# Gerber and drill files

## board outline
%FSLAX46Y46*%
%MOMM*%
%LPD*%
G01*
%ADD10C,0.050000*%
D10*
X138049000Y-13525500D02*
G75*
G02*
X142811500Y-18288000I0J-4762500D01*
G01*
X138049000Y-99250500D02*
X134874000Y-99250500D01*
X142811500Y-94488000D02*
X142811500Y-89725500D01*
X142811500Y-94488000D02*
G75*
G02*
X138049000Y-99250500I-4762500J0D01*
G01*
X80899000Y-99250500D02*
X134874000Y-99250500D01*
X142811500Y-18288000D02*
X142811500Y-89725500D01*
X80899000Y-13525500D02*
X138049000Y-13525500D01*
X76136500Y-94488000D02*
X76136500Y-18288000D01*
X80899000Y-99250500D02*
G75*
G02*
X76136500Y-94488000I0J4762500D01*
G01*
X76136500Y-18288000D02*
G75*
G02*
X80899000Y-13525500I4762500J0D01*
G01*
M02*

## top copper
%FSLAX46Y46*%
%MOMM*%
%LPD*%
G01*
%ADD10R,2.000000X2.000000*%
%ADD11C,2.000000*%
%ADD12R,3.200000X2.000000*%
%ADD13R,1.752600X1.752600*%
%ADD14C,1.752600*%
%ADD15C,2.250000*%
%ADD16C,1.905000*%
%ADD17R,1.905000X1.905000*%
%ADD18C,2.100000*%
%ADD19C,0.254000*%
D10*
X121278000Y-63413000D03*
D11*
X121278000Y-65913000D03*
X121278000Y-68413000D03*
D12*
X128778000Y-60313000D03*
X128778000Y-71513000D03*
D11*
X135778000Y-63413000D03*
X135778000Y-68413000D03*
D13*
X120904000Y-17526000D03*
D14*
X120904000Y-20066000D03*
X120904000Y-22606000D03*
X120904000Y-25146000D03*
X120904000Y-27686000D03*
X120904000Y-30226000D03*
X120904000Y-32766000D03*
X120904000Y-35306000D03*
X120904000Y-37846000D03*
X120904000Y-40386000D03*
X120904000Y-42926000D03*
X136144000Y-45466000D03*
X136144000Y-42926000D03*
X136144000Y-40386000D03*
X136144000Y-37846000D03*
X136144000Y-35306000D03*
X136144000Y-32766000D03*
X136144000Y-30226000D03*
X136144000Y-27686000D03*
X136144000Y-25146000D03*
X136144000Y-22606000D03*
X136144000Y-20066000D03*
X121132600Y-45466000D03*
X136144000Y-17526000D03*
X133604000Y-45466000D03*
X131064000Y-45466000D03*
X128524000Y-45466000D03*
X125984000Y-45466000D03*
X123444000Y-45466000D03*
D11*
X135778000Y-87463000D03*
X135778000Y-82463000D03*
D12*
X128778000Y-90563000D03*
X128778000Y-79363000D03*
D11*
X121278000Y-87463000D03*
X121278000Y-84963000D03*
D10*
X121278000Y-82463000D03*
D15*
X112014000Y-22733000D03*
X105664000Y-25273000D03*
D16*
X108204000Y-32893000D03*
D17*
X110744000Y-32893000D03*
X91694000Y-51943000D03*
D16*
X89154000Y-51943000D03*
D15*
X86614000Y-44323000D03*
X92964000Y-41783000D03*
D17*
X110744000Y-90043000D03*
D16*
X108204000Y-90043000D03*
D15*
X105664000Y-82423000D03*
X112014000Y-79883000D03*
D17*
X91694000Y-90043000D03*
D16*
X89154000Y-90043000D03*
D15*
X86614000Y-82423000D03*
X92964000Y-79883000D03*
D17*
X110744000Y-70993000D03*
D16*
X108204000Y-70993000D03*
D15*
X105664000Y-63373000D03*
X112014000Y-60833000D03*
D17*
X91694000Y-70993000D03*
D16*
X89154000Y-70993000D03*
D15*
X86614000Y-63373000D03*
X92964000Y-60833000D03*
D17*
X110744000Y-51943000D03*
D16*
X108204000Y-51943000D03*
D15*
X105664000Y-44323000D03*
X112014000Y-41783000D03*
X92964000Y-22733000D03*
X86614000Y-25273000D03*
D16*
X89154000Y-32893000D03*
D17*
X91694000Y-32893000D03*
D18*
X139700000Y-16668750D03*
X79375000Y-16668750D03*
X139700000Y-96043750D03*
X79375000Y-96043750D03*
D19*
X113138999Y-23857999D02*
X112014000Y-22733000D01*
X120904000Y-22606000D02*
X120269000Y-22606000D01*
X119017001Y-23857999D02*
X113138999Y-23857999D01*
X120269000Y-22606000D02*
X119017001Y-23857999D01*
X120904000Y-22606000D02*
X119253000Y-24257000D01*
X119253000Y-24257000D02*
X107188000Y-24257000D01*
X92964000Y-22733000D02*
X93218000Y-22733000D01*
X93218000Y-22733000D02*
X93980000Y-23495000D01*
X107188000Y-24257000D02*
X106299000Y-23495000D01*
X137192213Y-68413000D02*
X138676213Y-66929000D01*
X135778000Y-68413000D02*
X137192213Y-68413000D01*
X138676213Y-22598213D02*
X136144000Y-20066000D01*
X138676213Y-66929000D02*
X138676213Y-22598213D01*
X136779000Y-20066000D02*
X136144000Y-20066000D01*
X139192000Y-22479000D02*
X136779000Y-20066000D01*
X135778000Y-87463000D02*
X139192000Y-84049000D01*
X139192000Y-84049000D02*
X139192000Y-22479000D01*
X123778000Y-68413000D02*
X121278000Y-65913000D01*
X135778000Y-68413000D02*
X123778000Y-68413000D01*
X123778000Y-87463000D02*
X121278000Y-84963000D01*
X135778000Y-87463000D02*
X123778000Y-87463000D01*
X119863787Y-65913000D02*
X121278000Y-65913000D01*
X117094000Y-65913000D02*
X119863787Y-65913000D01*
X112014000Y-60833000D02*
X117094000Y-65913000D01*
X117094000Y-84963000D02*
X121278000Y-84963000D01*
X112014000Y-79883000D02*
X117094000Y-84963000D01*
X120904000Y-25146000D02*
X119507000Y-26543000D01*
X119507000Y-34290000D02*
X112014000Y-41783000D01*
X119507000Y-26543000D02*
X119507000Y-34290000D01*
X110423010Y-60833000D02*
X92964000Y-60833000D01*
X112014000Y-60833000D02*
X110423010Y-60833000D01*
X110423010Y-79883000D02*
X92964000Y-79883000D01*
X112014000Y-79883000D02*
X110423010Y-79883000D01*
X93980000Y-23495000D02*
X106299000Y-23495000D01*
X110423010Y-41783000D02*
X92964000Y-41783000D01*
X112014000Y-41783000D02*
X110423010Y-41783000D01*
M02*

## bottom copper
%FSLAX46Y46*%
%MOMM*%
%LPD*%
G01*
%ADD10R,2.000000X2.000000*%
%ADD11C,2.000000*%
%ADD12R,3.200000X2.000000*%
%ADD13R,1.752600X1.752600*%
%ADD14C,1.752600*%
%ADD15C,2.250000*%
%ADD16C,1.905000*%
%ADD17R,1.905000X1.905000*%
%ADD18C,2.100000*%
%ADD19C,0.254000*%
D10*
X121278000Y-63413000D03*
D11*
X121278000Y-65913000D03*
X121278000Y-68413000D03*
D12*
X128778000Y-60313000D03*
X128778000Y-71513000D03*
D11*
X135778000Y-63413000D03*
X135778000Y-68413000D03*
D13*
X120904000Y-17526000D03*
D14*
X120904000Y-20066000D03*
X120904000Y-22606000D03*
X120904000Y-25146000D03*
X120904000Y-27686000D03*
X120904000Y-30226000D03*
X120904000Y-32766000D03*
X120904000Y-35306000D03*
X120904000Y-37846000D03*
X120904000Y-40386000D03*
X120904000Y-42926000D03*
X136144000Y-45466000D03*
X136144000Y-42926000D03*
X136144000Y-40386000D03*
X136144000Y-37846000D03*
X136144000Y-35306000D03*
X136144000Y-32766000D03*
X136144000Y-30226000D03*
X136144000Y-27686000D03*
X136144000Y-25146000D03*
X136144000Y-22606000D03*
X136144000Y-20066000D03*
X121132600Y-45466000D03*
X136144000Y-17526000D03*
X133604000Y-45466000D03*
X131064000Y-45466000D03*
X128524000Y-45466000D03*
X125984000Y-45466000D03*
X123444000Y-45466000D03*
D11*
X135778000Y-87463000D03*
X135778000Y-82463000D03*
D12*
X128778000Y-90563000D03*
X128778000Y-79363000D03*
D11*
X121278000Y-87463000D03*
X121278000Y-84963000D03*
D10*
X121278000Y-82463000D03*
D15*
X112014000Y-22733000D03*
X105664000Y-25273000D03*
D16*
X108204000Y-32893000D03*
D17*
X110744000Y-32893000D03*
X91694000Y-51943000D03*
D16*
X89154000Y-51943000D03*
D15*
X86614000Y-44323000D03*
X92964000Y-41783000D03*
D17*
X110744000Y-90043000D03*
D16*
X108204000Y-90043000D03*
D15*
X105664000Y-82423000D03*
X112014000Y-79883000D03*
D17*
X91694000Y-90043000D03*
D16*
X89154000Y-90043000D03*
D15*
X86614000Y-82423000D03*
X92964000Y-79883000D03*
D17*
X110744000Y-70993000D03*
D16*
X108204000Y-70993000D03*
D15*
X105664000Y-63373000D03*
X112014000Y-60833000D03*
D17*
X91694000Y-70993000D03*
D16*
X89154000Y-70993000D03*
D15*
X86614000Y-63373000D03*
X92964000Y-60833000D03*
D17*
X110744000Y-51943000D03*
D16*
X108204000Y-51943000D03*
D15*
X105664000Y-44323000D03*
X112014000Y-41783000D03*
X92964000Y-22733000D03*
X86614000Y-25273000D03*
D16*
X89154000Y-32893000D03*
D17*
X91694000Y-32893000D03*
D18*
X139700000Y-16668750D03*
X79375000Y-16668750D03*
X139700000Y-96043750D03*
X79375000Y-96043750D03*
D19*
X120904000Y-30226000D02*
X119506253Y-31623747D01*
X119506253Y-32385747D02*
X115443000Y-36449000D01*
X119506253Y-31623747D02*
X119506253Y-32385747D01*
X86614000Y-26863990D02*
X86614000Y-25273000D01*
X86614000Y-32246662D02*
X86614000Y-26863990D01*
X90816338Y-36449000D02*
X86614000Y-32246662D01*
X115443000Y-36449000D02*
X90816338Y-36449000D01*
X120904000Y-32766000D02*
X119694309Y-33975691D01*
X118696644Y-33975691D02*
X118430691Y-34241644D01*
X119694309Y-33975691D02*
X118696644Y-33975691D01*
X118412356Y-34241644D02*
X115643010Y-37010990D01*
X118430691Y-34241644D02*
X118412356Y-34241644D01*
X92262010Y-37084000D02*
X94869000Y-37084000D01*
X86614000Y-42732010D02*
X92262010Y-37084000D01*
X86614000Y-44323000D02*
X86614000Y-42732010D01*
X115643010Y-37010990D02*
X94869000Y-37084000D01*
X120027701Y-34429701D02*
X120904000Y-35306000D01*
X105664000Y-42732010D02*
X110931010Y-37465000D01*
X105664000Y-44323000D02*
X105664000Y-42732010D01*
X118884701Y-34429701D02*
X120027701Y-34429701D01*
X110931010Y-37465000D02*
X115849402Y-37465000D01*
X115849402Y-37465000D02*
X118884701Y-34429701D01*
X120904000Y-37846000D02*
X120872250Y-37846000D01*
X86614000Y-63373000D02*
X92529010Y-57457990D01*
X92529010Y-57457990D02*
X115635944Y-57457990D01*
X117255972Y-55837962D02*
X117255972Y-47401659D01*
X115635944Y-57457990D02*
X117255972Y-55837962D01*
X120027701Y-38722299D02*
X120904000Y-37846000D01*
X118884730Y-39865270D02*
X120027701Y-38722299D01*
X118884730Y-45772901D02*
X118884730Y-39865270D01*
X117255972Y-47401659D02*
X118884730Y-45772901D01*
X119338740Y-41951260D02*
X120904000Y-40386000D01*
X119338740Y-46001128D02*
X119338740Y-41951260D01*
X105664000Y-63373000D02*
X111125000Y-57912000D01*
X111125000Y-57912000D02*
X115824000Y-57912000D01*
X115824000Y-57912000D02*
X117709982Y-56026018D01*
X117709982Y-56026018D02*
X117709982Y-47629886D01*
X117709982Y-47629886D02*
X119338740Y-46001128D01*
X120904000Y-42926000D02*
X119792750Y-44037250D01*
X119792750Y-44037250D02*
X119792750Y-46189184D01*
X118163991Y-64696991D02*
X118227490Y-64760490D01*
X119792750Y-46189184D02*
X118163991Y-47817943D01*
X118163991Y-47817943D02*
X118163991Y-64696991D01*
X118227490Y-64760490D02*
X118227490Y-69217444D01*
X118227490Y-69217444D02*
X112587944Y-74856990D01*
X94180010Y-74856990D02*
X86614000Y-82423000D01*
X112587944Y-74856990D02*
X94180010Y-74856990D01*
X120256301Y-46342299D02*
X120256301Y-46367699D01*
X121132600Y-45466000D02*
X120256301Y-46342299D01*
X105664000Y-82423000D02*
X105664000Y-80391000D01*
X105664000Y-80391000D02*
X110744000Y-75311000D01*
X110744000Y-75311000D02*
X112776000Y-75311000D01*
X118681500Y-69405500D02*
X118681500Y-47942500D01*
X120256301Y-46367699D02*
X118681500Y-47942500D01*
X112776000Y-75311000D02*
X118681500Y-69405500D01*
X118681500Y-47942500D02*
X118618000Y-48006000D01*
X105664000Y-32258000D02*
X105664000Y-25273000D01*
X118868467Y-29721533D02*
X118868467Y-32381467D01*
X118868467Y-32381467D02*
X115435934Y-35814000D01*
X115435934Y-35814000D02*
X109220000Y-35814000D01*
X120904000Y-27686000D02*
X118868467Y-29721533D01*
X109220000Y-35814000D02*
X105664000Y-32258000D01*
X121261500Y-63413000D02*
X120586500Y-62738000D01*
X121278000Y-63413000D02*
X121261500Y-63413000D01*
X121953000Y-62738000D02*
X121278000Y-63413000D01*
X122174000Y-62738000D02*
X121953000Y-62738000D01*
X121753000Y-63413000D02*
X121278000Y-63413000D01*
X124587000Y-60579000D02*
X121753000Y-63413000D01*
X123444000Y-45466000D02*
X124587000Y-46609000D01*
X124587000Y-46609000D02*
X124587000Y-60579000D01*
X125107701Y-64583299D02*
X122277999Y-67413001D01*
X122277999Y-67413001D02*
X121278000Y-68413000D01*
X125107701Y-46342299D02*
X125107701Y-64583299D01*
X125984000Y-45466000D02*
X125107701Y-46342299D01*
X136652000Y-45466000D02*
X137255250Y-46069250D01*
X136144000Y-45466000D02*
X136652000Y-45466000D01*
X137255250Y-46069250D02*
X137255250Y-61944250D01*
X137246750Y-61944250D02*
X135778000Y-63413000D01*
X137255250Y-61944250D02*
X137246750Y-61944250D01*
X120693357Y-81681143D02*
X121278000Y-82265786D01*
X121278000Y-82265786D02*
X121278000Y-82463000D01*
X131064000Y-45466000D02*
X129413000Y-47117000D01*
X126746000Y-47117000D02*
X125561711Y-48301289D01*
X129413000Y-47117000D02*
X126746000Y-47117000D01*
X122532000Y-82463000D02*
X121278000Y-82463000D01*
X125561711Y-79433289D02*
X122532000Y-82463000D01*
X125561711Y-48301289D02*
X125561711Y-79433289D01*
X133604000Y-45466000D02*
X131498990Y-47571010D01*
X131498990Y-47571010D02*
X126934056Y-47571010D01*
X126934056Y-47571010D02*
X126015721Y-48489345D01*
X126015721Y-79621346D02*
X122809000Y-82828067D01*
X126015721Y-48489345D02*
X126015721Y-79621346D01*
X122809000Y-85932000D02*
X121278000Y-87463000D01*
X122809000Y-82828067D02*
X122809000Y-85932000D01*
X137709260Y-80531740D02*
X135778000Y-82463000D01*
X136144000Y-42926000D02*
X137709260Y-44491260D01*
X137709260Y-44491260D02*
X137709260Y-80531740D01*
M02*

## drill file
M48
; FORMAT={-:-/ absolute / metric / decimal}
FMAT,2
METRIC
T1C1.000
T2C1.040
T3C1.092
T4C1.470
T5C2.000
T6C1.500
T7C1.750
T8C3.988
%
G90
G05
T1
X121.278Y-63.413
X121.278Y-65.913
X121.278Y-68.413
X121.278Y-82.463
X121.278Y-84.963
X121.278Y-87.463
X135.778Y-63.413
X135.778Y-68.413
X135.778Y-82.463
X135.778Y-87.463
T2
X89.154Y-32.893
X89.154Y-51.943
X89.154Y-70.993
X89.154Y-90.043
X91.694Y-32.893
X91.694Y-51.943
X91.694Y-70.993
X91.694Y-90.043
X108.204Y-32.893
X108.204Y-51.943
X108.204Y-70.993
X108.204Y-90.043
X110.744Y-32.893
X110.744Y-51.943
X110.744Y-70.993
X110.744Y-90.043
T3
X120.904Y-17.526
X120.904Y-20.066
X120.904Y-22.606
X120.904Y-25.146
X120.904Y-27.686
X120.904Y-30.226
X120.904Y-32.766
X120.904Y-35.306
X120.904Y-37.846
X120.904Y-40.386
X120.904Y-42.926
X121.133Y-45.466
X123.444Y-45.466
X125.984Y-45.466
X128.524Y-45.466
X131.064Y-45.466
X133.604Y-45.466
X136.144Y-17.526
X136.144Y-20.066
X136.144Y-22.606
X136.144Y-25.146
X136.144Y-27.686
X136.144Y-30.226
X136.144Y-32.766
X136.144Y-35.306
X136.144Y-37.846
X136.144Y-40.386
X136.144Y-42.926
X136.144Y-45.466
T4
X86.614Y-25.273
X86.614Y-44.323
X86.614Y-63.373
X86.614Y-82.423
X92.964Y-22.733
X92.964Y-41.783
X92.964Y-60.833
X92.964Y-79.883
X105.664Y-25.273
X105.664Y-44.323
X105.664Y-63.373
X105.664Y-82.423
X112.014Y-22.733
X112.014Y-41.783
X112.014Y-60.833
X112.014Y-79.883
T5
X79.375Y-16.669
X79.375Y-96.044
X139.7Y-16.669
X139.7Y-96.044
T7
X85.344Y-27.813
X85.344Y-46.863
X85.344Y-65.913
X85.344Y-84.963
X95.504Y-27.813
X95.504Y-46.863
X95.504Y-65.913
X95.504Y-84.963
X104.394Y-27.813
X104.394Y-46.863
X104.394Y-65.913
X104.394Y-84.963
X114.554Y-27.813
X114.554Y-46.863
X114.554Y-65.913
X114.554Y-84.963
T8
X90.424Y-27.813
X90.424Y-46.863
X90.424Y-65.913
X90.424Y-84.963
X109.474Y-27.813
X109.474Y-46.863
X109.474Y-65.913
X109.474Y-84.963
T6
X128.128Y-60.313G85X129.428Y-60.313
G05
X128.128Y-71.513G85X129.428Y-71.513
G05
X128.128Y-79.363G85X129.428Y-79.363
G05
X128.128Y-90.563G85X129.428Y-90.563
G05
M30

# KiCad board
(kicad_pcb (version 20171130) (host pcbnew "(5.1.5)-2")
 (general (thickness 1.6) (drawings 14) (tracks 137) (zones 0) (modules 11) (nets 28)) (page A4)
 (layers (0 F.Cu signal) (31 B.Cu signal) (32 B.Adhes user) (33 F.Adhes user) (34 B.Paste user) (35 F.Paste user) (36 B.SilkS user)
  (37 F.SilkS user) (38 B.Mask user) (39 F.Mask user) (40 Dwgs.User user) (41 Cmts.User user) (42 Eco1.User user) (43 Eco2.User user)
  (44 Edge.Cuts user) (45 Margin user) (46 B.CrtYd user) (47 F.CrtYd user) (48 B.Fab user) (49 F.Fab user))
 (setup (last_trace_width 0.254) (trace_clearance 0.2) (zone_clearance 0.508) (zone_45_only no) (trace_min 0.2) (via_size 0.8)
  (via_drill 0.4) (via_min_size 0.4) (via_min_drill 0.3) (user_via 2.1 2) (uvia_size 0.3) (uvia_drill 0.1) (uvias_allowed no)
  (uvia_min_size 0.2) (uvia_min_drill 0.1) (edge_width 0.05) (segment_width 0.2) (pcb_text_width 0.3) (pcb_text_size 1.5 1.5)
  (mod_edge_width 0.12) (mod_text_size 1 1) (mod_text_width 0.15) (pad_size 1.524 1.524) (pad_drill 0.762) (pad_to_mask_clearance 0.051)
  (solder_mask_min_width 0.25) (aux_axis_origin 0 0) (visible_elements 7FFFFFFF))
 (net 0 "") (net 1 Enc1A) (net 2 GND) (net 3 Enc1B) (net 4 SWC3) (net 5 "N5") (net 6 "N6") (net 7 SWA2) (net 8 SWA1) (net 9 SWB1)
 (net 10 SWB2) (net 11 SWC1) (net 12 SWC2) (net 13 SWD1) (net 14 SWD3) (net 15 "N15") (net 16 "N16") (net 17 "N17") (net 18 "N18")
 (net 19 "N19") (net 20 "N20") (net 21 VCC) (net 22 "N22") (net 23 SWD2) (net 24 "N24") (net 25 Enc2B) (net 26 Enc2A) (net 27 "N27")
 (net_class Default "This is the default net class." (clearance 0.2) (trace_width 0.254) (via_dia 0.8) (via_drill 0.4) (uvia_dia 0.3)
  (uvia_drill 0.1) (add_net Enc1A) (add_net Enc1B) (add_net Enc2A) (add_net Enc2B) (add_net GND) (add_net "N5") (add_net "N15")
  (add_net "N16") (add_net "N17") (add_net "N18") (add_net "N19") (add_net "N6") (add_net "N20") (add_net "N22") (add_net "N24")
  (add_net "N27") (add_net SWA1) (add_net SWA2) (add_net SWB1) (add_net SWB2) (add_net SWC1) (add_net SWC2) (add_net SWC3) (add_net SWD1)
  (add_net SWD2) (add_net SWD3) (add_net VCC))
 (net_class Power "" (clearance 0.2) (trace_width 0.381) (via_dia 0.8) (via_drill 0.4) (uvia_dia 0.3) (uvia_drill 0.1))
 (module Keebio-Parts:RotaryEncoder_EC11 (layer F.Cu) (at 128.778 65.913)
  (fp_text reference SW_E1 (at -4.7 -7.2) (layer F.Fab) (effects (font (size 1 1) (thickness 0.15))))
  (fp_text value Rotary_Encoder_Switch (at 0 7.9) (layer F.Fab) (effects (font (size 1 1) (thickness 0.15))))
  (pad A thru_hole rect (at -7.5 -2.5) (size 2 2) (drill 1) (layers *.Cu *.Mask) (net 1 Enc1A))
  (pad C thru_hole circle (at -7.5 0) (size 2 2) (drill 1) (layers *.Cu *.Mask) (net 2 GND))
  (pad B thru_hole circle (at -7.5 2.5) (size 2 2) (drill 1) (layers *.Cu *.Mask) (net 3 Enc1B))
  (pad "" np_thru_hole rect (at 0 -5.6) (size 3.2 2) (drill oval 2.8 1.5) (layers *.Cu *.Mask))
  (pad "" np_thru_hole rect (at 0 5.6) (size 3.2 2) (drill oval 2.8 1.5) (layers *.Cu *.Mask))
  (pad S2 thru_hole circle (at 7 -2.5) (size 2 2) (drill 1) (layers *.Cu *.Mask) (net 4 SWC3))
  (pad S1 thru_hole circle (at 7 2.5) (size 2 2) (drill 1) (layers *.Cu *.Mask) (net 2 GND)))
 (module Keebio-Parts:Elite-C (layer F.Cu) (at 128.524 31.496 270)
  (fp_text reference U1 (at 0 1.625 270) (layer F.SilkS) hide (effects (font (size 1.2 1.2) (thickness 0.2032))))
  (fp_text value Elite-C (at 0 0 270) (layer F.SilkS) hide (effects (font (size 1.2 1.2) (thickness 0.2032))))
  (pad 1 thru_hole rect (at -13.97 7.62 270) (size 1.7526 1.7526) (drill 1.0922) (layers *.Cu *.SilkS *.Mask) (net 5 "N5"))
  (pad 2 thru_hole circle (at -11.43 7.62 270) (size 1.7526 1.7526) (drill 1.0922) (layers *.Cu *.SilkS *.Mask) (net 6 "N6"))
  (pad 3 thru_hole circle (at -8.89 7.62 270) (size 1.7526 1.7526) (drill 1.0922) (layers *.Cu *.SilkS *.Mask) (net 2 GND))
  (pad 4 thru_hole circle (at -6.35 7.62 270) (size 1.7526 1.7526) (drill 1.0922) (layers *.Cu *.SilkS *.Mask) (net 2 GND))
  (pad 5 thru_hole circle (at -3.81 7.62 270) (size 1.7526 1.7526) (drill 1.0922) (layers *.Cu *.SilkS *.Mask) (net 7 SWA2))
  (pad 6 thru_hole circle (at -1.27 7.62 270) (size 1.7526 1.7526) (drill 1.0922) (layers *.Cu *.SilkS *.Mask) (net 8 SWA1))
  (pad 7 thru_hole circle (at 1.27 7.62 270) (size 1.7526 1.7526) (drill 1.0922) (layers *.Cu *.SilkS *.Mask) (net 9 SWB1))
  (pad 8 thru_hole circle (at 3.81 7.62 270) (size 1.7526 1.7526) (drill 1.0922) (layers *.Cu *.SilkS *.Mask) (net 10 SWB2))
  (pad 9 thru_hole circle (at 6.35 7.62 270) (size 1.7526 1.7526) (drill 1.0922) (layers *.Cu *.SilkS *.Mask) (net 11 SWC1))
  (pad 10 thru_hole circle (at 8.89 7.62 270) (size 1.7526 1.7526) (drill 1.0922) (layers *.Cu *.SilkS *.Mask) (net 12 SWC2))
  (pad 11 thru_hole circle (at 11.43 7.62 270) (size 1.7526 1.7526) (drill 1.0922) (layers *.Cu *.SilkS *.Mask) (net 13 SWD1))
  (pad 13 thru_hole circle (at 13.97 -7.62 270) (size 1.7526 1.7526) (drill 1.0922) (layers *.Cu *.SilkS *.Mask) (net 4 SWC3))
  (pad 14 thru_hole circle (at 11.43 -7.62 270) (size 1.7526 1.7526) (drill 1.0922) (layers *.Cu *.SilkS *.Mask) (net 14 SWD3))
  (pad 15 thru_hole circle (at 8.89 -7.62 270) (size 1.7526 1.7526) (drill 1.0922) (layers *.Cu *.SilkS *.Mask) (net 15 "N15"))
  (pad 16 thru_hole circle (at 6.35 -7.62 270) (size 1.7526 1.7526) (drill 1.0922) (layers *.Cu *.SilkS *.Mask) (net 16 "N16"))
  (pad 17 thru_hole circle (at 3.81 -7.62 270) (size 1.7526 1.7526) (drill 1.0922) (layers *.Cu *.SilkS *.Mask) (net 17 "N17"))
  (pad 18 thru_hole circle (at 1.27 -7.62 270) (size 1.7526 1.7526) (drill 1.0922) (layers *.Cu *.SilkS *.Mask) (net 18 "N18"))
  (pad 19 thru_hole circle (at -1.27 -7.62 270) (size 1.7526 1.7526) (drill 1.0922) (layers *.Cu *.SilkS *.Mask) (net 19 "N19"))
  (pad 20 thru_hole circle (at -3.81 -7.62 270) (size 1.7526 1.7526) (drill 1.0922) (layers *.Cu *.SilkS *.Mask) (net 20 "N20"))
  (pad 21 thru_hole circle (at -6.35 -7.62 270) (size 1.7526 1.7526) (drill 1.0922) (layers *.Cu *.SilkS *.Mask) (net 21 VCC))
  (pad 22 thru_hole circle (at -8.89 -7.62 270) (size 1.7526 1.7526) (drill 1.0922) (layers *.Cu *.SilkS *.Mask) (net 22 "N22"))
  (pad 23 thru_hole circle (at -11.43 -7.62 270) (size 1.7526 1.7526) (drill 1.0922) (layers *.Cu *.SilkS *.Mask) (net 2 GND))
  (pad 12 thru_hole circle (at 13.97 7.3914 270) (size 1.7526 1.7526) (drill 1.0922) (layers *.Cu *.SilkS *.Mask) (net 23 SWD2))
  (pad 24 thru_hole circle (at -13.97 -7.62 270) (size 1.7526 1.7526) (drill 1.0922) (layers *.Cu *.SilkS *.Mask) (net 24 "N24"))
  (pad 29 thru_hole circle (at 13.97 -5.08 270) (size 1.7526 1.7526) (drill 1.0922) (layers *.Cu *.SilkS *.Mask) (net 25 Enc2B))
  (pad 28 thru_hole circle (at 13.97 -2.54 270) (size 1.7526 1.7526) (drill 1.0922) (layers *.Cu *.SilkS *.Mask) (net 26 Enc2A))
  (pad 27 thru_hole circle (at 13.97 0 270) (size 1.7526 1.7526) (drill 1.0922) (layers *.Cu *.SilkS *.Mask) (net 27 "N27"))
  (pad 26 thru_hole circle (at 13.97 2.54 270) (size 1.7526 1.7526) (drill 1.0922) (layers *.Cu *.SilkS *.Mask) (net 3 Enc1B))
  (pad 25 thru_hole circle (at 13.97 5.08 270) (size 1.7526 1.7526) (drill 1.0922) (layers *.Cu *.SilkS *.Mask) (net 1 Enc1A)))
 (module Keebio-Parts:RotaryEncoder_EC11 (layer F.Cu) (at 128.778 84.963)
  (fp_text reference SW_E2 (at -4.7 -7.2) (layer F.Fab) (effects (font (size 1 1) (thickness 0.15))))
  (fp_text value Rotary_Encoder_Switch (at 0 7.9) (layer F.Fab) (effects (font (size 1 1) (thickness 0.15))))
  (pad S1 thru_hole circle (at 7 2.5) (size 2 2) (drill 1) (layers *.Cu *.Mask) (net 2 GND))
  (pad S2 thru_hole circle (at 7 -2.5) (size 2 2) (drill 1) (layers *.Cu *.Mask) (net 14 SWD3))
  (pad "" np_thru_hole rect (at 0 5.6) (size 3.2 2) (drill oval 2.8 1.5) (layers *.Cu *.Mask))
  (pad "" np_thru_hole rect (at 0 -5.6) (size 3.2 2) (drill oval 2.8 1.5) (layers *.Cu *.Mask))
  (pad B thru_hole circle (at -7.5 2.5) (size 2 2) (drill 1) (layers *.Cu *.Mask) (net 25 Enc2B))
  (pad C thru_hole circle (at -7.5 0) (size 2 2) (drill 1) (layers *.Cu *.Mask) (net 2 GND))
  (pad A thru_hole rect (at -7.5 -2.5) (size 2 2) (drill 1) (layers *.Cu *.Mask) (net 26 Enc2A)))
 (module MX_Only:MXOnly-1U (layer F.Cu) (at 109.474 27.813)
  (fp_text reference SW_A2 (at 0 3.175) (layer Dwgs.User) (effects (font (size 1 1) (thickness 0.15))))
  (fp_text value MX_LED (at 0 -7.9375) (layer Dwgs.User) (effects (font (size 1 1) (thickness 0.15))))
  (pad 2 thru_hole circle (at 2.54 -5.08) (size 2.25 2.25) (drill 1.47) (layers *.Cu B.Mask) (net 2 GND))
  (pad "" np_thru_hole circle (at 0 0) (size 3.9878 3.9878) (drill 3.9878) (layers *.Cu *.Mask))
  (pad 1 thru_hole circle (at -3.81 -2.54) (size 2.25 2.25) (drill 1.47) (layers *.Cu B.Mask) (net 7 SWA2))
  (pad 3 thru_hole circle (at -1.27 5.08) (size 1.905 1.905) (drill 1.04) (layers *.Cu B.Mask))
  (pad 4 thru_hole rect (at 1.27 5.08) (size 1.905 1.905) (drill 1.04) (layers *.Cu B.Mask))
  (pad "" np_thru_hole circle (at -5.08 0 48.0996) (size 1.75 1.75) (drill 1.75) (layers *.Cu *.Mask))
  (pad "" np_thru_hole circle (at 5.08 0 48.0996) (size 1.75 1.75) (drill 1.75) (layers *.Cu *.Mask)))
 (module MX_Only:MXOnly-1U (layer F.Cu) (at 90.424 46.863)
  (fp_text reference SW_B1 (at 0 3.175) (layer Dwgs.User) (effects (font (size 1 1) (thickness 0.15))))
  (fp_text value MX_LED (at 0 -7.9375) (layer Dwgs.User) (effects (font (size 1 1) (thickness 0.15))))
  (pad "" np_thru_hole circle (at 5.08 0 48.0996) (size 1.75 1.75) (drill 1.75) (layers *.Cu *.Mask))
  (pad "" np_thru_hole circle (at -5.08 0 48.0996) (size 1.75 1.75) (drill 1.75) (layers *.Cu *.Mask))
  (pad 4 thru_hole rect (at 1.27 5.08) (size 1.905 1.905) (drill 1.04) (layers *.Cu B.Mask))
  (pad 3 thru_hole circle (at -1.27 5.08) (size 1.905 1.905) (drill 1.04) (layers *.Cu B.Mask))
  (pad 1 thru_hole circle (at -3.81 -2.54) (size 2.25 2.25) (drill 1.47) (layers *.Cu B.Mask) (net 9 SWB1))
  (pad "" np_thru_hole circle (at 0 0) (size 3.9878 3.9878) (drill 3.9878) (layers *.Cu *.Mask))
  (pad 2 thru_hole circle (at 2.54 -5.08) (size 2.25 2.25) (drill 1.47) (layers *.Cu B.Mask) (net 2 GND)))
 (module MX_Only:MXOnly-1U (layer F.Cu) (at 109.474 84.963)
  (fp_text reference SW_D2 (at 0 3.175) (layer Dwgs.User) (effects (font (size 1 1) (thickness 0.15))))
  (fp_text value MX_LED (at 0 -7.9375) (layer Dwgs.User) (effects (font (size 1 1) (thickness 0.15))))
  (pad "" np_thru_hole circle (at 5.08 0 48.0996) (size 1.75 1.75) (drill 1.75) (layers *.Cu *.Mask))
  (pad "" np_thru_hole circle (at -5.08 0 48.0996) (size 1.75 1.75) (drill 1.75) (layers *.Cu *.Mask))
  (pad 4 thru_hole rect (at 1.27 5.08) (size 1.905 1.905) (drill 1.04) (layers *.Cu B.Mask))
  (pad 3 thru_hole circle (at -1.27 5.08) (size 1.905 1.905) (drill 1.04) (layers *.Cu B.Mask))
  (pad 1 thru_hole circle (at -3.81 -2.54) (size 2.25 2.25) (drill 1.47) (layers *.Cu B.Mask) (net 23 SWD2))
  (pad "" np_thru_hole circle (at 0 0) (size 3.9878 3.9878) (drill 3.9878) (layers *.Cu *.Mask))
  (pad 2 thru_hole circle (at 2.54 -5.08) (size 2.25 2.25) (drill 1.47) (layers *.Cu B.Mask) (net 2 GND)))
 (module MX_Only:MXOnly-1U (layer F.Cu) (at 90.424 84.963)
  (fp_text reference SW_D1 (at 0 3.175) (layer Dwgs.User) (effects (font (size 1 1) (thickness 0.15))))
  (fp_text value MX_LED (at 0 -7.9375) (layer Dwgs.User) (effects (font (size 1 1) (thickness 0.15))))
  (pad "" np_thru_hole circle (at 5.08 0 48.0996) (size 1.75 1.75) (drill 1.75) (layers *.Cu *.Mask))
  (pad "" np_thru_hole circle (at -5.08 0 48.0996) (size 1.75 1.75) (drill 1.75) (layers *.Cu *.Mask))
  (pad 4 thru_hole rect (at 1.27 5.08) (size 1.905 1.905) (drill 1.04) (layers *.Cu B.Mask))
  (pad 3 thru_hole circle (at -1.27 5.08) (size 1.905 1.905) (drill 1.04) (layers *.Cu B.Mask))
  (pad 1 thru_hole circle (at -3.81 -2.54) (size 2.25 2.25) (drill 1.47) (layers *.Cu B.Mask) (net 13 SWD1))
  (pad "" np_thru_hole circle (at 0 0) (size 3.9878 3.9878) (drill 3.9878) (layers *.Cu *.Mask))
  (pad 2 thru_hole circle (at 2.54 -5.08) (size 2.25 2.25) (drill 1.47) (layers *.Cu B.Mask) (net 2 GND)))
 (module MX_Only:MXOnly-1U (layer F.Cu) (at 109.474 65.913)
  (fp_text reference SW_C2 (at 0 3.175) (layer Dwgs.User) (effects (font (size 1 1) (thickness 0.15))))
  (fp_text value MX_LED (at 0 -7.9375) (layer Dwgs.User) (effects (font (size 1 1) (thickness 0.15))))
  (pad "" np_thru_hole circle (at 5.08 0 48.0996) (size 1.75 1.75) (drill 1.75) (layers *.Cu *.Mask))
  (pad "" np_thru_hole circle (at -5.08 0 48.0996) (size 1.75 1.75) (drill 1.75) (layers *.Cu *.Mask))
  (pad 4 thru_hole rect (at 1.27 5.08) (size 1.905 1.905) (drill 1.04) (layers *.Cu B.Mask))
  (pad 3 thru_hole circle (at -1.27 5.08) (size 1.905 1.905) (drill 1.04) (layers *.Cu B.Mask))
  (pad 1 thru_hole circle (at -3.81 -2.54) (size 2.25 2.25) (drill 1.47) (layers *.Cu B.Mask) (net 12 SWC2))
  (pad "" np_thru_hole circle (at 0 0) (size 3.9878 3.9878) (drill 3.9878) (layers *.Cu *.Mask))
  (pad 2 thru_hole circle (at 2.54 -5.08) (size 2.25 2.25) (drill 1.47) (layers *.Cu B.Mask) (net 2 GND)))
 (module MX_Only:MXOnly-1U (layer F.Cu) (at 90.424 65.913)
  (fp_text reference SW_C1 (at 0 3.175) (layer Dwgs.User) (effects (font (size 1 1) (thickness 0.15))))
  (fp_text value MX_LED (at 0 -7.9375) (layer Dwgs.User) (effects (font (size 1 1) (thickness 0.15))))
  (pad "" np_thru_hole circle (at 5.08 0 48.0996) (size 1.75 1.75) (drill 1.75) (layers *.Cu *.Mask))
  (pad "" np_thru_hole circle (at -5.08 0 48.0996) (size 1.75 1.75) (drill 1.75) (layers *.Cu *.Mask))
  (pad 4 thru_hole rect (at 1.27 5.08) (size 1.905 1.905) (drill 1.04) (layers *.Cu B.Mask))
  (pad 3 thru_hole circle (at -1.27 5.08) (size 1.905 1.905) (drill 1.04) (layers *.Cu B.Mask))
  (pad 1 thru_hole circle (at -3.81 -2.54) (size 2.25 2.25) (drill 1.47) (layers *.Cu B.Mask) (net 11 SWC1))
  (pad "" np_thru_hole circle (at 0 0) (size 3.9878 3.9878) (drill 3.9878) (layers *.Cu *.Mask))
  (pad 2 thru_hole circle (at 2.54 -5.08) (size 2.25 2.25) (drill 1.47) (layers *.Cu B.Mask) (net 2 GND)))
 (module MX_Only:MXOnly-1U (layer F.Cu) (at 109.474 46.863)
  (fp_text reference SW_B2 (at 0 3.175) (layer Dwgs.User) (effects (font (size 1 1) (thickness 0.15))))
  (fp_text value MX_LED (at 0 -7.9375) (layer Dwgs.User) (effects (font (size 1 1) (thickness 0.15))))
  (pad "" np_thru_hole circle (at 5.08 0 48.0996) (size 1.75 1.75) (drill 1.75) (layers *.Cu *.Mask))
  (pad "" np_thru_hole circle (at -5.08 0 48.0996) (size 1.75 1.75) (drill 1.75) (layers *.Cu *.Mask))
  (pad 4 thru_hole rect (at 1.27 5.08) (size 1.905 1.905) (drill 1.04) (layers *.Cu B.Mask))
  (pad 3 thru_hole circle (at -1.27 5.08) (size 1.905 1.905) (drill 1.04) (layers *.Cu B.Mask))
  (pad 1 thru_hole circle (at -3.81 -2.54) (size 2.25 2.25) (drill 1.47) (layers *.Cu B.Mask) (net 10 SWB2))
  (pad "" np_thru_hole circle (at 0 0) (size 3.9878 3.9878) (drill 3.9878) (layers *.Cu *.Mask))
  (pad 2 thru_hole circle (at 2.54 -5.08) (size 2.25 2.25) (drill 1.47) (layers *.Cu B.Mask) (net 2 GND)))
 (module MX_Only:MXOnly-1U (layer F.Cu) (at 90.424 27.813)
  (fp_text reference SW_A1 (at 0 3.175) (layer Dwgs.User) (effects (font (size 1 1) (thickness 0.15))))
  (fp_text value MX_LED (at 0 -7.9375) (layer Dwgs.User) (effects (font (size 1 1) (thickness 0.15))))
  (pad 2 thru_hole circle (at 2.54 -5.08) (size 2.25 2.25) (drill 1.47) (layers *.Cu B.Mask) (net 2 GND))
  (pad "" np_thru_hole circle (at 0 0) (size 3.9878 3.9878) (drill 3.9878) (layers *.Cu *.Mask))
  (pad 1 thru_hole circle (at -3.81 -2.54) (size 2.25 2.25) (drill 1.47) (layers *.Cu B.Mask) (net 8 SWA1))
  (pad 3 thru_hole circle (at -1.27 5.08) (size 1.905 1.905) (drill 1.04) (layers *.Cu B.Mask))
  (pad 4 thru_hole rect (at 1.27 5.08) (size 1.905 1.905) (drill 1.04) (layers *.Cu B.Mask))
  (pad "" np_thru_hole circle (at -5.08 0 48.0996) (size 1.75 1.75) (drill 1.75) (layers *.Cu *.Mask))
  (pad "" np_thru_hole circle (at 5.08 0 48.0996) (size 1.75 1.75) (drill 1.75) (layers *.Cu *.Mask)))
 (gr_arc (start 138.049 18.288) (end 142.8115 18.288) (angle -90) (layer Edge.Cuts) (width 0.05))
 (gr_line (start 138.049 99.2505) (end 134.874 99.2505) (layer Edge.Cuts) (width 0.05))
 (gr_line (start 142.8115 94.488) (end 142.8115 89.7255) (layer Edge.Cuts) (width 0.05))
 (gr_arc (start 138.049 94.488) (end 138.049 99.2505) (angle -90) (layer Edge.Cuts) (width 0.05))
 (gr_line (start 80.899 99.2505) (end 134.874 99.2505) (layer Edge.Cuts) (width 0.05))
 (gr_line (start 142.8115 18.288) (end 142.8115 89.7255) (layer Edge.Cuts) (width 0.05))
 (gr_line (start 80.899 13.5255) (end 138.049 13.5255) (layer Edge.Cuts) (width 0.05))
 (gr_line (start 76.1365 94.488) (end 76.1365 18.288) (layer Edge.Cuts) (width 0.05))
 (gr_arc (start 80.899 94.488) (end 76.1365 94.488) (angle -90) (layer Edge.Cuts) (width 0.05))
 (gr_arc (start 80.899 18.288) (end 80.899 13.5255) (angle -90) (layer Edge.Cuts) (width 0.05))
 (via (at 139.7 16.66875) (size 2.1) (drill 2) (layers F.Cu B.Cu) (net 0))
 (via (at 79.375 16.66875) (size 2.1) (drill 2) (layers F.Cu B.Cu) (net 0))
 (via (at 139.7 96.04375) (size 2.1) (drill 2) (layers F.Cu B.Cu) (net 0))
 (via (at 79.375 96.04375) (size 2.1) (drill 2) (layers F.Cu B.Cu) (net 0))
 (segment (start 120.904 30.226) (end 119.506253 31.623747) (width 0.254) (layer B.Cu) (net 8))
 (segment (start 119.506253 32.385747) (end 115.443 36.449) (width 0.254) (layer B.Cu) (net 8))
 (segment (start 119.506253 31.623747) (end 119.506253 32.385747) (width 0.254) (layer B.Cu) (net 8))
 (segment (start 86.614 26.86399) (end 86.614 25.273) (width 0.254) (layer B.Cu) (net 8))
 (segment (start 86.614 32.246662) (end 86.614 26.86399) (width 0.254) (layer B.Cu) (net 8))
 (segment (start 90.816338 36.449) (end 86.614 32.246662) (width 0.254) (layer B.Cu) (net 8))
 (segment (start 115.443 36.449) (end 90.816338 36.449) (width 0.254) (layer B.Cu) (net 8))
 (segment (start 113.138999 23.857999) (end 112.014 22.733) (width 0.254) (layer F.Cu) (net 2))
 (segment (start 120.904 22.606) (end 120.269 22.606) (width 0.254) (layer F.Cu) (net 2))
 (segment (start 119.017001 23.857999) (end 113.138999 23.857999) (width 0.254) (layer F.Cu) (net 2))
 (segment (start 120.269 22.606) (end 119.017001 23.857999) (width 0.254) (layer F.Cu) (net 2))
 (segment (start 120.904 22.606) (end 119.253 24.257) (width 0.254) (layer F.Cu) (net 2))
 (segment (start 119.253 24.257) (end 107.188 24.257) (width 0.254) (layer F.Cu) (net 2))
 (segment (start 92.964 22.733) (end 93.218 22.733) (width 0.254) (layer F.Cu) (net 2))
 (segment (start 93.218 22.733) (end 93.98 23.495) (width 0.254) (layer F.Cu) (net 2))
 (segment (start 107.188 24.257) (end 106.299 23.495) (width 0.254) (layer F.Cu) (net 2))
 (segment (start 137.192213 68.413) (end 138.676213 66.929) (width 0.254) (layer F.Cu) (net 2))
 (segment (start 135.778 68.413) (end 137.192213 68.413) (width 0.254) (layer F.Cu) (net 2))
 (segment (start 138.676213 22.598213) (end 136.144 20.066) (width 0.254) (layer F.Cu) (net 2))
 (segment (start 138.676213 66.929) (end 138.676213 22.598213) (width 0.254) (layer F.Cu) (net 2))
 (segment (start 136.779 20.066) (end 136.144 20.066) (width 0.254) (layer F.Cu) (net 2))
 (segment (start 139.192 22.479) (end 136.779 20.066) (width 0.254) (layer F.Cu) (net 2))
 (segment (start 135.778 87.463) (end 139.192 84.049) (width 0.254) (layer F.Cu) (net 2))
 (segment (start 139.192 84.049) (end 139.192 22.479) (width 0.254) (layer F.Cu) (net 2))
 (segment (start 123.778 68.413) (end 121.278 65.913) (width 0.254) (layer F.Cu) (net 2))
 (segment (start 135.778 68.413) (end 123.778 68.413) (width 0.254) (layer F.Cu) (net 2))
 (segment (start 123.778 87.463) (end 121.278 84.963) (width 0.254) (layer F.Cu) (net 2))
 (segment (start 135.778 87.463) (end 123.778 87.463) (width 0.254) (layer F.Cu) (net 2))
 (segment (start 119.863787 65.913) (end 121.278 65.913) (width 0.254) (layer F.Cu) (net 2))
 (segment (start 117.094 65.913) (end 119.863787 65.913) (width 0.254) (layer F.Cu) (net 2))
 (segment (start 112.014 60.833) (end 117.094 65.913) (width 0.254) (layer F.Cu) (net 2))
 (segment (start 117.094 84.963) (end 121.278 84.963) (width 0.254) (layer F.Cu) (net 2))
 (segment (start 112.014 79.883) (end 117.094 84.963) (width 0.254) (layer F.Cu) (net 2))
 (segment (start 120.904 25.146) (end 119.507 26.543) (width 0.254) (layer F.Cu) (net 2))
 (segment (start 119.507 34.29) (end 112.014 41.783) (width 0.254) (layer F.Cu) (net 2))
 (segment (start 119.507 26.543) (end 119.507 34.29) (width 0.254) (layer F.Cu) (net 2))
 (segment (start 110.42301 60.833) (end 92.964 60.833) (width 0.254) (layer F.Cu) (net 2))
 (segment (start 112.014 60.833) (end 110.42301 60.833) (width 0.254) (layer F.Cu) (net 2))
 (segment (start 110.42301 79.883) (end 92.964 79.883) (width 0.254) (layer F.Cu) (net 2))
 (segment (start 112.014 79.883) (end 110.42301 79.883) (width 0.254) (layer F.Cu) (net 2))
 (segment (start 93.98 23.495) (end 106.299 23.495) (width 0.254) (layer F.Cu) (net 2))
 (segment (start 110.42301 41.783) (end 92.964 41.783) (width 0.254) (layer F.Cu) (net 2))
 (segment (start 112.014 41.783) (end 110.42301 41.783) (width 0.254) (layer F.Cu) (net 2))
 (segment (start 120.904 32.766) (end 119.694309 33.975691) (width 0.254) (layer B.Cu) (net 9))
 (segment (start 118.696644 33.975691) (end 118.430691 34.241644) (width 0.254) (layer B.Cu) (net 9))
 (segment (start 119.694309 33.975691) (end 118.696644 33.975691) (width 0.254) (layer B.Cu) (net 9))
 (segment (start 118.412356 34.241644) (end 115.64301 37.01099) (width 0.254) (layer B.Cu) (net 9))
 (segment (start 118.430691 34.241644) (end 118.412356 34.241644) (width 0.254) (layer B.Cu) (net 9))
 (segment (start 92.26201 37.084) (end 94.869 37.084) (width 0.254) (layer B.Cu) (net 9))
 (segment (start 86.614 42.73201) (end 92.26201 37.084) (width 0.254) (layer B.Cu) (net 9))
 (segment (start 86.614 44.323) (end 86.614 42.73201) (width 0.254) (layer B.Cu) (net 9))
 (segment (start 115.64301 37.01099) (end 94.869 37.084) (width 0.254) (layer B.Cu) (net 9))
 (segment (start 120.027701 34.429701) (end 120.904 35.306) (width 0.254) (layer B.Cu) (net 10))
 (segment (start 105.664 42.73201) (end 110.93101 37.465) (width 0.254) (layer B.Cu) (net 10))
 (segment (start 105.664 44.323) (end 105.664 42.73201) (width 0.254) (layer B.Cu) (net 10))
 (segment (start 118.884701 34.429701) (end 120.027701 34.429701) (width 0.254) (layer B.Cu) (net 10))
 (segment (start 110.93101 37.465) (end 115.849402 37.465) (width 0.254) (layer B.Cu) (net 10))
 (segment (start 115.849402 37.465) (end 118.884701 34.429701) (width 0.254) (layer B.Cu) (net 10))
 (segment (start 120.904 37.846) (end 120.87225 37.846) (width 0.254) (layer B.Cu) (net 11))
 (segment (start 86.614 63.373) (end 92.52901 57.45799) (width 0.254) (layer B.Cu) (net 11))
 (segment (start 92.52901 57.45799) (end 115.635944 57.45799) (width 0.254) (layer B.Cu) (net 11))
 (segment (start 117.255972 55.837962) (end 117.255972 47.401659) (width 0.254) (layer B.Cu) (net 11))
 (segment (start 115.635944 57.45799) (end 117.255972 55.837962) (width 0.254) (layer B.Cu) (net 11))
 (segment (start 120.027701 38.722299) (end 120.904 37.846) (width 0.254) (layer B.Cu) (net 11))
 (segment (start 118.88473 39.86527) (end 120.027701 38.722299) (width 0.254) (layer B.Cu) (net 11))
 (segment (start 118.88473 45.772901) (end 118.88473 39.86527) (width 0.254) (layer B.Cu) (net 11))
 (segment (start 117.255972 47.401659) (end 118.88473 45.772901) (width 0.254) (layer B.Cu) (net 11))
 (segment (start 119.33874 41.95126) (end 120.904 40.386) (width 0.254) (layer B.Cu) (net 12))
 (segment (start 119.33874 46.001128) (end 119.33874 41.95126) (width 0.254) (layer B.Cu) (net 12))
 (segment (start 105.664 63.373) (end 111.125 57.912) (width 0.254) (layer B.Cu) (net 12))
 (segment (start 111.125 57.912) (end 115.824 57.912) (width 0.254) (layer B.Cu) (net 12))
 (segment (start 115.824 57.912) (end 117.709982 56.026018) (width 0.254) (layer B.Cu) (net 12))
 (segment (start 117.709982 56.026018) (end 117.709982 47.629886) (width 0.254) (layer B.Cu) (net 12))
 (segment (start 117.709982 47.629886) (end 119.33874 46.001128) (width 0.254) (layer B.Cu) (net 12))
 (segment (start 120.904 42.926) (end 119.79275 44.03725) (width 0.254) (layer B.Cu) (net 13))
 (segment (start 119.79275 44.03725) (end 119.79275 46.189184) (width 0.254) (layer B.Cu) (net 13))
 (segment (start 118.163991 64.696991) (end 118.22749 64.76049) (width 0.254) (layer B.Cu) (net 13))
 (segment (start 119.79275 46.189184) (end 118.163991 47.817943) (width 0.254) (layer B.Cu) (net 13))
 (segment (start 118.163991 47.817943) (end 118.163991 64.696991) (width 0.254) (layer B.Cu) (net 13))
 (segment (start 118.22749 64.76049) (end 118.22749 69.217444) (width 0.254) (layer B.Cu) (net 13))
 (segment (start 118.22749 69.217444) (end 112.587944 74.85699) (width 0.254) (layer B.Cu) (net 13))
 (segment (start 94.18001 74.85699) (end 86.614 82.423) (width 0.254) (layer B.Cu) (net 13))
 (segment (start 112.587944 74.85699) (end 94.18001 74.85699) (width 0.254) (layer B.Cu) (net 13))
 (segment (start 120.256301 46.342299) (end 120.256301 46.367699) (width 0.254) (layer B.Cu) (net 23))
 (segment (start 121.1326 45.466) (end 120.256301 46.342299) (width 0.254) (layer B.Cu) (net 23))
 (segment (start 105.664 82.423) (end 105.664 80.391) (width 0.254) (layer B.Cu) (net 23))
 (segment (start 105.664 80.391) (end 110.744 75.311) (width 0.254) (layer B.Cu) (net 23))
 (segment (start 110.744 75.311) (end 112.776 75.311) (width 0.254) (layer B.Cu) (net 23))
 (segment (start 118.6815 69.4055) (end 118.6815 47.9425) (width 0.254) (layer B.Cu) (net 23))
 (segment (start 120.256301 46.367699) (end 118.6815 47.9425) (width 0.254) (layer B.Cu) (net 23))
 (segment (start 112.776 75.311) (end 118.6815 69.4055) (width 0.254) (layer B.Cu) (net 23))
 (segment (start 118.6815 47.9425) (end 118.618 48.006) (width 0.254) (layer B.Cu) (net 23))
 (segment (start 105.664 32.258) (end 105.664 25.273) (width 0.254) (layer B.Cu) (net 7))
 (segment (start 118.868467 29.721533) (end 118.868467 32.381467) (width 0.254) (layer B.Cu) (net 7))
 (segment (start 118.868467 32.381467) (end 115.435934 35.814) (width 0.254) (layer B.Cu) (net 7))
 (segment (start 115.435934 35.814) (end 109.22 35.814) (width 0.254) (layer B.Cu) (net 7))
 (segment (start 120.904 27.686) (end 118.868467 29.721533) (width 0.254) (layer B.Cu) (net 7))
 (segment (start 109.22 35.814) (end 105.664 32.258) (width 0.254) (layer B.Cu) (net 7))
 (segment (start 121.2615 63.413) (end 120.5865 62.738) (width 0.254) (layer B.Cu) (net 1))
 (segment (start 121.278 63.413) (end 121.2615 63.413) (width 0.254) (layer B.Cu) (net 1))
 (segment (start 121.953 62.738) (end 121.278 63.413) (width 0.254) (layer B.Cu) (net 1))
 (segment (start 122.174 62.738) (end 121.953 62.738) (width 0.254) (layer B.Cu) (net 1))
 (segment (start 121.753 63.413) (end 121.278 63.413) (width 0.254) (layer B.Cu) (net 1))
 (segment (start 124.587 60.579) (end 121.753 63.413) (width 0.254) (layer B.Cu) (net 1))
 (segment (start 123.444 45.466) (end 124.587 46.609) (width 0.254) (layer B.Cu) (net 1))
 (segment (start 124.587 46.609) (end 124.587 60.579) (width 0.254) (layer B.Cu) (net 1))
 (segment (start 125.107701 64.583299) (end 122.277999 67.413001) (width 0.254) (layer B.Cu) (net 3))
 (segment (start 122.277999 67.413001) (end 121.278 68.413) (width 0.254) (layer B.Cu) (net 3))
 (segment (start 125.107701 46.342299) (end 125.107701 64.583299) (width 0.254) (layer B.Cu) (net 3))
 (segment (start 125.984 45.466) (end 125.107701 46.342299) (width 0.254) (layer B.Cu) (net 3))
 (segment (start 136.652 45.466) (end 137.25525 46.06925) (width 0.254) (layer B.Cu) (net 4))
 (segment (start 136.144 45.466) (end 136.652 45.466) (width 0.254) (layer B.Cu) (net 4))
 (segment (start 137.25525 46.06925) (end 137.25525 61.94425) (width 0.254) (layer B.Cu) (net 4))
 (segment (start 137.24675 61.94425) (end 135.778 63.413) (width 0.254) (layer B.Cu) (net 4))
 (segment (start 137.25525 61.94425) (end 137.24675 61.94425) (width 0.254) (layer B.Cu) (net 4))
 (segment (start 120.693357 81.681143) (end 121.278 82.265786) (width 0.254) (layer B.Cu) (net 26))
 (segment (start 121.278 82.265786) (end 121.278 82.463) (width 0.254) (layer B.Cu) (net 26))
 (segment (start 131.064 45.466) (end 129.413 47.117) (width 0.254) (layer B.Cu) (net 26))
 (segment (start 126.746 47.117) (end 125.561711 48.301289) (width 0.254) (layer B.Cu) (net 26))
 (segment (start 129.413 47.117) (end 126.746 47.117) (width 0.254) (layer B.Cu) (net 26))
 (segment (start 122.532 82.463) (end 121.278 82.463) (width 0.254) (layer B.Cu) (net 26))
 (segment (start 125.561711 79.433289) (end 122.532 82.463) (width 0.254) (layer B.Cu) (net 26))
 (segment (start 125.561711 48.301289) (end 125.561711 79.433289) (width 0.254) (layer B.Cu) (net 26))
 (segment (start 133.604 45.466) (end 131.49899 47.57101) (width 0.254) (layer B.Cu) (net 25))
 (segment (start 131.49899 47.57101) (end 126.934056 47.57101) (width 0.254) (layer B.Cu) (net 25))
 (segment (start 126.934056 47.57101) (end 126.015721 48.489345) (width 0.254) (layer B.Cu) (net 25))
 (segment (start 126.015721 79.621346) (end 122.809 82.828067) (width 0.254) (layer B.Cu) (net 25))
 (segment (start 126.015721 48.489345) (end 126.015721 79.621346) (width 0.254) (layer B.Cu) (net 25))
 (segment (start 122.809 85.932) (end 121.278 87.463) (width 0.254) (layer B.Cu) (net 25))
 (segment (start 122.809 82.828067) (end 122.809 85.932) (width 0.254) (layer B.Cu) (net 25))
 (segment (start 137.70926 80.53174) (end 135.778 82.463) (width 0.254) (layer B.Cu) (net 14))
 (segment (start 136.144 42.926) (end 137.70926 44.49126) (width 0.254) (layer B.Cu) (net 14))
 (segment (start 137.70926 44.49126) (end 137.70926 80.53174) (width 0.254) (layer B.Cu) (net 14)))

